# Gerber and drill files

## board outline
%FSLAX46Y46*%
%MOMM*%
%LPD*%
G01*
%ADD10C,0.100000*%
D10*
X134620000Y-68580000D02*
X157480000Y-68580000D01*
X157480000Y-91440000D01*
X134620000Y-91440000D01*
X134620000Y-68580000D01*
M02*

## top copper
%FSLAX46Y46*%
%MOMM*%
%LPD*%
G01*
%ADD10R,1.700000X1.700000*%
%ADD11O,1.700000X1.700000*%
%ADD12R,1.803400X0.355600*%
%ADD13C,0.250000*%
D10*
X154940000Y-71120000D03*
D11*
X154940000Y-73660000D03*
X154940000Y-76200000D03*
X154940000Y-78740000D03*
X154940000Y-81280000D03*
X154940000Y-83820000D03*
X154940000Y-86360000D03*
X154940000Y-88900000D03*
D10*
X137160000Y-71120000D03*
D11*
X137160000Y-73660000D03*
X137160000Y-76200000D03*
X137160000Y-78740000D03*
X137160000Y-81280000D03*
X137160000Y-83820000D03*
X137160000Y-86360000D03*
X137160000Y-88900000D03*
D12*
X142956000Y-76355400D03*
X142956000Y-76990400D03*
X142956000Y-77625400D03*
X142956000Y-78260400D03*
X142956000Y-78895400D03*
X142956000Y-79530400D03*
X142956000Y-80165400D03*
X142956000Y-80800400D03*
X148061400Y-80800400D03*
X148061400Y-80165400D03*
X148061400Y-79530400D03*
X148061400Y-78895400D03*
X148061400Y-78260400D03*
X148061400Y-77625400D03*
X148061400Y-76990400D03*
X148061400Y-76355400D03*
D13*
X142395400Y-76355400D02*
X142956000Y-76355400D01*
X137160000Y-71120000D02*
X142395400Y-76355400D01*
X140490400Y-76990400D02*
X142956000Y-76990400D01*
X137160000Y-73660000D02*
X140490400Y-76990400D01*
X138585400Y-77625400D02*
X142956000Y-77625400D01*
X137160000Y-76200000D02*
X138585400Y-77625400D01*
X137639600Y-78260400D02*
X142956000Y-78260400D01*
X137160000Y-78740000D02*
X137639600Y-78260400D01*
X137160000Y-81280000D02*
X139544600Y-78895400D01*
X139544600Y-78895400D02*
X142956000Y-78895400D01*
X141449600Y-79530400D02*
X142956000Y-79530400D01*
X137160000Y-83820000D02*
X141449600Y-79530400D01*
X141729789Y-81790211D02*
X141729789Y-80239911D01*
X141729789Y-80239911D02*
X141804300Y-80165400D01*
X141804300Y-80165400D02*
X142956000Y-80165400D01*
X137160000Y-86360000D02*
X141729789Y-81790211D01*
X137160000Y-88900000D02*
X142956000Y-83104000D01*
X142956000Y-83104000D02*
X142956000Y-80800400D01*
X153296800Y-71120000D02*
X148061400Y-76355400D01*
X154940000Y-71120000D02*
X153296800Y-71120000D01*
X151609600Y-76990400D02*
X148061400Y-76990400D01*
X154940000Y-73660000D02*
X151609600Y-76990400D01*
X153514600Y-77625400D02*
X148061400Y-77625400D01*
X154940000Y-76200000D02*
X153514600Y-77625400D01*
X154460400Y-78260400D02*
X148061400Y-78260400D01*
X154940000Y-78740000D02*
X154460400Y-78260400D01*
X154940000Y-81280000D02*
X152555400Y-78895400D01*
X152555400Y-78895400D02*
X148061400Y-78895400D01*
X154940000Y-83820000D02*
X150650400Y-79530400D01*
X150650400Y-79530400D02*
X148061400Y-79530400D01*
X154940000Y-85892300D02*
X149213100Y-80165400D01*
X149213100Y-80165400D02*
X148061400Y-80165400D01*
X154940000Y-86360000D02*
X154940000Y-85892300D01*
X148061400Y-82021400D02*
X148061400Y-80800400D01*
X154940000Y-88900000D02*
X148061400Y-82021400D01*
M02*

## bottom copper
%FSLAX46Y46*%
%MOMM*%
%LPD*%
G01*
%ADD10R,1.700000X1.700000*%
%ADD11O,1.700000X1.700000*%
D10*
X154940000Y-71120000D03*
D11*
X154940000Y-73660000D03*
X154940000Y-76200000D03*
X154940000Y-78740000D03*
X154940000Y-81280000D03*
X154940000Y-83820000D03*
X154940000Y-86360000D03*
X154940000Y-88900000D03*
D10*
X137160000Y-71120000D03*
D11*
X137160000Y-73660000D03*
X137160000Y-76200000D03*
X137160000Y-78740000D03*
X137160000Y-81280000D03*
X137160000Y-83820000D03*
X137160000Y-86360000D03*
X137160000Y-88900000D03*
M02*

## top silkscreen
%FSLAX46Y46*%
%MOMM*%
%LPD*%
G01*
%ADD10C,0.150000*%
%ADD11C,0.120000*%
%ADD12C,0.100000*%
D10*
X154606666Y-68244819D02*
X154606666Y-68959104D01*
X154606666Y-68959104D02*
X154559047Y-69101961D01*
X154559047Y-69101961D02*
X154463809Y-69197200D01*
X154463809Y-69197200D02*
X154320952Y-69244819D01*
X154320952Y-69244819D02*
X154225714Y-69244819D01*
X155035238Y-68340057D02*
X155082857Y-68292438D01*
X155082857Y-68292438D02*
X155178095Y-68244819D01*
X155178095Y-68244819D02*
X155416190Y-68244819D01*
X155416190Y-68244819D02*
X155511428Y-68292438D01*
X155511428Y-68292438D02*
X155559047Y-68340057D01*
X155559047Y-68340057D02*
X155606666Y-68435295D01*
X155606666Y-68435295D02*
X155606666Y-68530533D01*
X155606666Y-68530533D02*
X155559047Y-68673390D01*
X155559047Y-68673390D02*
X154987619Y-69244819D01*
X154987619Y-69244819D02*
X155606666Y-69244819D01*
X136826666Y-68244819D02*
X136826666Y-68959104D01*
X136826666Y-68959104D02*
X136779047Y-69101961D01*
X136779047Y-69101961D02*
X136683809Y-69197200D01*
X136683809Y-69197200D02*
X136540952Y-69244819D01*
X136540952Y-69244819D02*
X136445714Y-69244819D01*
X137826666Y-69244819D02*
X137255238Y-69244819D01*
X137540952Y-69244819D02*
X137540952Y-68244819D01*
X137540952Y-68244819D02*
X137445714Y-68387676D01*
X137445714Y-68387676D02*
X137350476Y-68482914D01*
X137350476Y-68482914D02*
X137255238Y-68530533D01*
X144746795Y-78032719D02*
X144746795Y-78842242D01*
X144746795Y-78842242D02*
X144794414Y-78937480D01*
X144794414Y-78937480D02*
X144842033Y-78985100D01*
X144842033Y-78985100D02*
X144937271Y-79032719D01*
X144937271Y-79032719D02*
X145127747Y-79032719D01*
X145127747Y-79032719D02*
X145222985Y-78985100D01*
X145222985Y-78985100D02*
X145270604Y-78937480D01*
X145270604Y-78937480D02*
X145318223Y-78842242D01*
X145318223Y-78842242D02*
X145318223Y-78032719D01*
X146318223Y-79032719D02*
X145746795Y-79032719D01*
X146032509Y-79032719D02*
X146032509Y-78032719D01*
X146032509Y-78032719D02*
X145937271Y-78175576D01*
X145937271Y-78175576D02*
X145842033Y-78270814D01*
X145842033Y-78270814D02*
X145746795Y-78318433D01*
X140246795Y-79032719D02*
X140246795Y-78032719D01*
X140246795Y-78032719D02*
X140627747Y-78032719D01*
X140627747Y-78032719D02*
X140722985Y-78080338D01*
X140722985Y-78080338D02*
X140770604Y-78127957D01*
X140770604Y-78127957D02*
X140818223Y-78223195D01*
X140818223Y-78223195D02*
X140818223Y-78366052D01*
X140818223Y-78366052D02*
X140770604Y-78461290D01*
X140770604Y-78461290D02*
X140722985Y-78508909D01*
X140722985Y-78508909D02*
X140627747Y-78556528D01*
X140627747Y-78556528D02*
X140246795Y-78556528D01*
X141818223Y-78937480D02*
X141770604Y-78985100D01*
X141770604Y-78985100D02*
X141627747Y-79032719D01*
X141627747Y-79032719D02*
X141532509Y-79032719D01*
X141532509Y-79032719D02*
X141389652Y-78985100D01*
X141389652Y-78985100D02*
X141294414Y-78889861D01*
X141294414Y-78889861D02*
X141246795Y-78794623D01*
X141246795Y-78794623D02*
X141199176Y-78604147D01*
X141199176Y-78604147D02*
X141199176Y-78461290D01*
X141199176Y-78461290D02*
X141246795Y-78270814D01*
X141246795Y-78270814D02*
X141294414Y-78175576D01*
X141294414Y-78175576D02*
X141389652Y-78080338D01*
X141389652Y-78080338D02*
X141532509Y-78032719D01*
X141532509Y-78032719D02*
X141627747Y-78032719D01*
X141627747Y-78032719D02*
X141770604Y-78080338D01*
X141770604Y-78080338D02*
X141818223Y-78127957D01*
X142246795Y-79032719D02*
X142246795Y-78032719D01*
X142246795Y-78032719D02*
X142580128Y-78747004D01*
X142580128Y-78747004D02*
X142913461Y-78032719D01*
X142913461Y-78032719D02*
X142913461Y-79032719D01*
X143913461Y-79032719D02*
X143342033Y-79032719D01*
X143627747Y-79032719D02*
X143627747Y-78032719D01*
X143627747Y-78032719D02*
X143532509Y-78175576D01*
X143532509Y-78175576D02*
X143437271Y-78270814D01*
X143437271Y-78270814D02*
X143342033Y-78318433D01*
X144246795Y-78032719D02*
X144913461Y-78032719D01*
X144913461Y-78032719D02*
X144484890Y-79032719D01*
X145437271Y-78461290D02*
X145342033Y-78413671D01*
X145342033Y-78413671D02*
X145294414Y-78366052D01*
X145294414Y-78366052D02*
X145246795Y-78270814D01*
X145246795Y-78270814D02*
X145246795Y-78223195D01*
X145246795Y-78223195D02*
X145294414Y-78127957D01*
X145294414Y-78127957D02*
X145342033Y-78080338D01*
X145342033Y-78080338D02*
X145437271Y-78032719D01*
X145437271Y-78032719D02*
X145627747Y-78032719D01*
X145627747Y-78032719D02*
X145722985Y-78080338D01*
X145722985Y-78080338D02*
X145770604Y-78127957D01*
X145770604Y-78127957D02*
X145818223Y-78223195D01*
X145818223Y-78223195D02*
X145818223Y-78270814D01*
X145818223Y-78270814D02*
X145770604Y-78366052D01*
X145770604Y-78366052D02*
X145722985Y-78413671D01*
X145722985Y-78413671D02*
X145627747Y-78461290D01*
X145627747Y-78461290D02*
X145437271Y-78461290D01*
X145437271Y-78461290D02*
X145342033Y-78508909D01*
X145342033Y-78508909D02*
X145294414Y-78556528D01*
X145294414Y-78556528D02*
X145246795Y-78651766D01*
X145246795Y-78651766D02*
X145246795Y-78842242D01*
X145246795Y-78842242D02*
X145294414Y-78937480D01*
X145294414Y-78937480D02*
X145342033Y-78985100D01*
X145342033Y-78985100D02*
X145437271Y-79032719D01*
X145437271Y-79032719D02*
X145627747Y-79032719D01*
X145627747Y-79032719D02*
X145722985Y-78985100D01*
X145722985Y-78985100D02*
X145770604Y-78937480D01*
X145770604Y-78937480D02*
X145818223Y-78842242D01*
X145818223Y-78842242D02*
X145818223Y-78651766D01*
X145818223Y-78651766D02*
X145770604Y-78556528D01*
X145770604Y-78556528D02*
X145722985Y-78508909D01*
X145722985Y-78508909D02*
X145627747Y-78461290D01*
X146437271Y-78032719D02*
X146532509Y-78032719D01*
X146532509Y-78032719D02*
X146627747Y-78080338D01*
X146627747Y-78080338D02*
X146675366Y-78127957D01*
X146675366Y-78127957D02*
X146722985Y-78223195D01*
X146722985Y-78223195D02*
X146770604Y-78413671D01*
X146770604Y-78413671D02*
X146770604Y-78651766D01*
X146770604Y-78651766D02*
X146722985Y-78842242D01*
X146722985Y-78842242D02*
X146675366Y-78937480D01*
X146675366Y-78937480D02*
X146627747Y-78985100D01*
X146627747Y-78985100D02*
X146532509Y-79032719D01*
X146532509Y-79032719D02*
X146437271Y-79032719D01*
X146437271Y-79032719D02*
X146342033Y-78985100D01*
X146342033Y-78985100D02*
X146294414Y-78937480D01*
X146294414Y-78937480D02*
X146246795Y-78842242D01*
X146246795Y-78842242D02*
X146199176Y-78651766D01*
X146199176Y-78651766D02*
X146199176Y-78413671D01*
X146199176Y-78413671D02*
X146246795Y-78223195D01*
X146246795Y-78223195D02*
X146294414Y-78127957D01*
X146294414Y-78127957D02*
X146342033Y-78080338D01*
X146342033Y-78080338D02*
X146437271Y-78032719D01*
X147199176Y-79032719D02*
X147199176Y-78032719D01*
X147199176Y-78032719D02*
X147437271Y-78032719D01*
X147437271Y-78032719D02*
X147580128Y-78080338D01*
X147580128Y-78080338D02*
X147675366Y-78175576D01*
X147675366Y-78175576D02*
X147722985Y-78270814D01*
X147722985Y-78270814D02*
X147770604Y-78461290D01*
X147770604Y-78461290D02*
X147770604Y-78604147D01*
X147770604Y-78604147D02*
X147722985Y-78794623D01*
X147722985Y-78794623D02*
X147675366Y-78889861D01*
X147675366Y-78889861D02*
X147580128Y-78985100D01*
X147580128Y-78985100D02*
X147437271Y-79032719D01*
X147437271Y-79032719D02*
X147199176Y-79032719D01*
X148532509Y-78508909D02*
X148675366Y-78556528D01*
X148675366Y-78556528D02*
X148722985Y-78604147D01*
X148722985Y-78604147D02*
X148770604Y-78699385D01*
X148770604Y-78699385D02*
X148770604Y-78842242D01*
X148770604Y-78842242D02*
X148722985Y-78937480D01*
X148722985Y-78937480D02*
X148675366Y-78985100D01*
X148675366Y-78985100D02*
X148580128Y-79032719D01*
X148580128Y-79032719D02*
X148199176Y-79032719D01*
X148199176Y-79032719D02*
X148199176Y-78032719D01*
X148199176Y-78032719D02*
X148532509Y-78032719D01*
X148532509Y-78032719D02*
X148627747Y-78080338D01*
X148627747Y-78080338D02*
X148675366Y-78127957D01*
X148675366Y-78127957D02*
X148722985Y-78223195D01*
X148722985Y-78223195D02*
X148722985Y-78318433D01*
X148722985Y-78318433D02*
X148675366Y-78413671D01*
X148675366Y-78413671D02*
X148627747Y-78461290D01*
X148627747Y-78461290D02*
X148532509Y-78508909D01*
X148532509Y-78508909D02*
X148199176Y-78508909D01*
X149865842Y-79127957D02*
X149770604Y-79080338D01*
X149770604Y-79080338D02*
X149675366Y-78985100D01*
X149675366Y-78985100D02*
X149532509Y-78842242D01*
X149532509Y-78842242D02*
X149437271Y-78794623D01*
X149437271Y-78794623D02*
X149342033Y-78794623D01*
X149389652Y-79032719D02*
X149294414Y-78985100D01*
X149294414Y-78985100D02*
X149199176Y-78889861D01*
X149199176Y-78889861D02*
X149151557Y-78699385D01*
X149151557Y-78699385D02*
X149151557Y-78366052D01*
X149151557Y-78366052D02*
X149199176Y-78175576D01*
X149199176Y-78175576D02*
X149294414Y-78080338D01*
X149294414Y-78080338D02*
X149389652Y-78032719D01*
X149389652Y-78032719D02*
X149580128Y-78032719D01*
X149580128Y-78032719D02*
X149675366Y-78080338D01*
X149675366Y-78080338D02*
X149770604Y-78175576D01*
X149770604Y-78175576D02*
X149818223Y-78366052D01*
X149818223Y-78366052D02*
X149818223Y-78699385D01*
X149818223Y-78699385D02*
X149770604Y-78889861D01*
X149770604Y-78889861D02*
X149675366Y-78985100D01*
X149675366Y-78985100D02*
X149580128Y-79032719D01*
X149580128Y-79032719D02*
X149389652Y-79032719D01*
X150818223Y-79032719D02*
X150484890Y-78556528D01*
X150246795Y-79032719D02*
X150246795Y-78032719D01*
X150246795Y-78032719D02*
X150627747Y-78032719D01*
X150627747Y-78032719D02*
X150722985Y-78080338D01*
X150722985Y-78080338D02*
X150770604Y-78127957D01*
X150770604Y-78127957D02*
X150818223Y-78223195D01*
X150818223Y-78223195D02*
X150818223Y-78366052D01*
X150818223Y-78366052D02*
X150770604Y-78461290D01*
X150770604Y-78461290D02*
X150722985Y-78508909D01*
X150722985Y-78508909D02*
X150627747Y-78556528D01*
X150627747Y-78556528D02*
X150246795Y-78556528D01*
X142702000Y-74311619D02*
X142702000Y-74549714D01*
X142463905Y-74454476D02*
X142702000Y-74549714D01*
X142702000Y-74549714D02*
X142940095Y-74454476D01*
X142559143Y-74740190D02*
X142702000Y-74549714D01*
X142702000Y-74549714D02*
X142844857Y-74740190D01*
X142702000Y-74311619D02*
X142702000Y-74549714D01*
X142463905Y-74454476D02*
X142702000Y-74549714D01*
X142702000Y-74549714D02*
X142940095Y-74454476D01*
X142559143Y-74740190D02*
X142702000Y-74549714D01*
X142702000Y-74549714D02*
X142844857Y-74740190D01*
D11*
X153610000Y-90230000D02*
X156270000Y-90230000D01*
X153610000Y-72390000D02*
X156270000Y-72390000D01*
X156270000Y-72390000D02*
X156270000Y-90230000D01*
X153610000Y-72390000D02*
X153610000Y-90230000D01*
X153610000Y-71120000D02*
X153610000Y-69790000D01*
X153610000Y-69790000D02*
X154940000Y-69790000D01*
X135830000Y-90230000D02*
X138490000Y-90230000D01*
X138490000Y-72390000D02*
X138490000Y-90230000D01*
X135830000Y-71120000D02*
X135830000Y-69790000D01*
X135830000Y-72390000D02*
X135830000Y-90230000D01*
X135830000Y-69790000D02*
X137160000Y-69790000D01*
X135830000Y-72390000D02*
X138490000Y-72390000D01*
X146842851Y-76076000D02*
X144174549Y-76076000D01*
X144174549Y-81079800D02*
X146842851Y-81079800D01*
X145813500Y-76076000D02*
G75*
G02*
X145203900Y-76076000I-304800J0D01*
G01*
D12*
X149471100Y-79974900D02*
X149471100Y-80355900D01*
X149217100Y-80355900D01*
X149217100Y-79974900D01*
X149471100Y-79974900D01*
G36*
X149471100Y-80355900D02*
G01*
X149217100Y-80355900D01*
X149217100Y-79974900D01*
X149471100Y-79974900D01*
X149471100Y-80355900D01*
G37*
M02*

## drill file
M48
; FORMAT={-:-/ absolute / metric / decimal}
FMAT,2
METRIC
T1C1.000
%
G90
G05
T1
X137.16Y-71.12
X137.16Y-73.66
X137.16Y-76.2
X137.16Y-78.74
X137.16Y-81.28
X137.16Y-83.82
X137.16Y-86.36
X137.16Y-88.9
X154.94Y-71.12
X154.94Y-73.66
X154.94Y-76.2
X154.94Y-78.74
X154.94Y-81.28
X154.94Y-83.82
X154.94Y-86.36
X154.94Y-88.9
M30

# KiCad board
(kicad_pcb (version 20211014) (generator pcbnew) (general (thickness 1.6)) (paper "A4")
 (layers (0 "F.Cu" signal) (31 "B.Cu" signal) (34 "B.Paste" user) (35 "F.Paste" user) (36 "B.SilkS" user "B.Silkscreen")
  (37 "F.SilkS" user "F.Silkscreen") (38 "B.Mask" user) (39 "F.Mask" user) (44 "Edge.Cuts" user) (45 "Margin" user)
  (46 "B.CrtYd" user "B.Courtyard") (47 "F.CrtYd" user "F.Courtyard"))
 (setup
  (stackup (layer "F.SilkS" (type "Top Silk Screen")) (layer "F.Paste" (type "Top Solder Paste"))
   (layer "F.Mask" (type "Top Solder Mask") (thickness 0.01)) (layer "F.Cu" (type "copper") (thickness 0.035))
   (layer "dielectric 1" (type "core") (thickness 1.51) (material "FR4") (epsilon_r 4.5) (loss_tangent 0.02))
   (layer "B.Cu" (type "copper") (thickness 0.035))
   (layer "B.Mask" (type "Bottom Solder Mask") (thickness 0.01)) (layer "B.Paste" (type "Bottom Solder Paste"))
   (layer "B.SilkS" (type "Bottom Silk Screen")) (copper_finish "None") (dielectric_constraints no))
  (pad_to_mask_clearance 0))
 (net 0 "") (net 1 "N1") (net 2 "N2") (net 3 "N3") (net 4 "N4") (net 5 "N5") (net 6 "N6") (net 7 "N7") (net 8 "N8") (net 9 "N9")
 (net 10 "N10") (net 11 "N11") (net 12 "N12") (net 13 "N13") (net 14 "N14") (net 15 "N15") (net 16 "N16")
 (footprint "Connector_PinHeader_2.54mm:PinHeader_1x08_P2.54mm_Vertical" (layer "F.Cu") (at 154.94 71.12)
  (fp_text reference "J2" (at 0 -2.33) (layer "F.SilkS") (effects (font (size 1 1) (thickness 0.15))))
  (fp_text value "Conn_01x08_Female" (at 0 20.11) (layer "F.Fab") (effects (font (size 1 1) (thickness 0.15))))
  (fp_line (start -1.33 19.11) (end 1.33 19.11) (layer "F.SilkS") (width 0.12))
  (fp_line (start -1.33 1.27) (end 1.33 1.27) (layer "F.SilkS") (width 0.12))
  (fp_line (start 1.33 1.27) (end 1.33 19.11) (layer "F.SilkS") (width 0.12))
  (fp_line (start -1.33 1.27) (end -1.33 19.11) (layer "F.SilkS") (width 0.12))
  (fp_line (start -1.33 0) (end -1.33 -1.33) (layer "F.SilkS") (width 0.12))
  (fp_line (start -1.33 -1.33) (end 0 -1.33) (layer "F.SilkS") (width 0.12))
  (pad "1" thru_hole rect (at 0 0) (size 1.7 1.7) (drill 1) (layers *.Cu *.Mask) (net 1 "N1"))
  (pad "2" thru_hole oval (at 0 2.54) (size 1.7 1.7) (drill 1) (layers *.Cu *.Mask) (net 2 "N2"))
  (pad "3" thru_hole oval (at 0 5.08) (size 1.7 1.7) (drill 1) (layers *.Cu *.Mask) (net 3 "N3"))
  (pad "4" thru_hole oval (at 0 7.62) (size 1.7 1.7) (drill 1) (layers *.Cu *.Mask) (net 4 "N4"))
  (pad "5" thru_hole oval (at 0 10.16) (size 1.7 1.7) (drill 1) (layers *.Cu *.Mask) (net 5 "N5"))
  (pad "6" thru_hole oval (at 0 12.7) (size 1.7 1.7) (drill 1) (layers *.Cu *.Mask) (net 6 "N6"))
  (pad "7" thru_hole oval (at 0 15.24) (size 1.7 1.7) (drill 1) (layers *.Cu *.Mask) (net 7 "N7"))
  (pad "8" thru_hole oval (at 0 17.78) (size 1.7 1.7) (drill 1) (layers *.Cu *.Mask) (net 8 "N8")))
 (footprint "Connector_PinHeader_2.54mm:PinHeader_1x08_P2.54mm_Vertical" (layer "F.Cu") (at 137.16 71.12)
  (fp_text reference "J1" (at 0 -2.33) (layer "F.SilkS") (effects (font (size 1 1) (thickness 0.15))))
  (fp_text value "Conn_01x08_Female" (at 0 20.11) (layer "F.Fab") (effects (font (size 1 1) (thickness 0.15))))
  (fp_line (start -1.33 19.11) (end 1.33 19.11) (layer "F.SilkS") (width 0.12))
  (fp_line (start 1.33 1.27) (end 1.33 19.11) (layer "F.SilkS") (width 0.12))
  (fp_line (start -1.33 0) (end -1.33 -1.33) (layer "F.SilkS") (width 0.12))
  (fp_line (start -1.33 1.27) (end -1.33 19.11) (layer "F.SilkS") (width 0.12))
  (fp_line (start -1.33 -1.33) (end 0 -1.33) (layer "F.SilkS") (width 0.12))
  (fp_line (start -1.33 1.27) (end 1.33 1.27) (layer "F.SilkS") (width 0.12))
  (pad "1" thru_hole rect (at 0 0) (size 1.7 1.7) (drill 1) (layers *.Cu *.Mask) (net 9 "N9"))
  (pad "2" thru_hole oval (at 0 2.54) (size 1.7 1.7) (drill 1) (layers *.Cu *.Mask) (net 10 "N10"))
  (pad "3" thru_hole oval (at 0 5.08) (size 1.7 1.7) (drill 1) (layers *.Cu *.Mask) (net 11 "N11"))
  (pad "4" thru_hole oval (at 0 7.62) (size 1.7 1.7) (drill 1) (layers *.Cu *.Mask) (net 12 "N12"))
  (pad "5" thru_hole oval (at 0 10.16) (size 1.7 1.7) (drill 1) (layers *.Cu *.Mask) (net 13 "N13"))
  (pad "6" thru_hole oval (at 0 12.7) (size 1.7 1.7) (drill 1) (layers *.Cu *.Mask) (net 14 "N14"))
  (pad "7" thru_hole oval (at 0 15.24) (size 1.7 1.7) (drill 1) (layers *.Cu *.Mask) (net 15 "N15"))
  (pad "8" thru_hole oval (at 0 17.78) (size 1.7 1.7) (drill 1) (layers *.Cu *.Mask) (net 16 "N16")))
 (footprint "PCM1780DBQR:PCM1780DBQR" (layer "F.Cu") (at 145.5087 78.5779)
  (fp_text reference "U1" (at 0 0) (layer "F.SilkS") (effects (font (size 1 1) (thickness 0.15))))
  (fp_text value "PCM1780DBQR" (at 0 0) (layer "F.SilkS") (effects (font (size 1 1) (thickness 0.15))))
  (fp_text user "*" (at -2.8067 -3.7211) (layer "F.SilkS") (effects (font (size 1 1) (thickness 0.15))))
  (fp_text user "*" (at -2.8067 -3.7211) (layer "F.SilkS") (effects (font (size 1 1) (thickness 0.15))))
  (fp_line (start 1.334151 -2.5019) (end -1.334151 -2.5019) (layer "F.SilkS") (width 0.12))
  (fp_line (start -1.334151 2.5019) (end 1.334151 2.5019) (layer "F.SilkS") (width 0.12))
  (fp_arc (start 0.3048 -2.5019) (mid 0 -2.1971) (end -0.3048 -2.5019) (layer "F.SilkS") (width 0.12))
  (fp_poly (pts (xy 3.9624 1.397) (xy 3.9624 1.778) (xy 3.7084 1.778) (xy 3.7084 1.397)) (layer "F.SilkS") (width 0.1) (fill solid))
  (pad "1" smd rect (at -2.5527 -2.2225) (size 1.8034 0.3556) (layers "F.Cu" "F.Paste" "F.Mask") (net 9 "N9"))
  (pad "2" smd rect (at -2.5527 -1.5875) (size 1.8034 0.3556) (layers "F.Cu" "F.Paste" "F.Mask") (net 10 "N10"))
  (pad "3" smd rect (at -2.5527 -0.9525) (size 1.8034 0.3556) (layers "F.Cu" "F.Paste" "F.Mask") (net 11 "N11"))
  (pad "4" smd rect (at -2.5527 -0.3175) (size 1.8034 0.3556) (layers "F.Cu" "F.Paste" "F.Mask") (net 12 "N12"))
  (pad "5" smd rect (at -2.5527 0.3175) (size 1.8034 0.3556) (layers "F.Cu" "F.Paste" "F.Mask") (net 13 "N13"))
  (pad "6" smd rect (at -2.5527 0.9525) (size 1.8034 0.3556) (layers "F.Cu" "F.Paste" "F.Mask") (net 14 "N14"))
  (pad "7" smd rect (at -2.5527 1.5875) (size 1.8034 0.3556) (layers "F.Cu" "F.Paste" "F.Mask") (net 15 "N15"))
  (pad "8" smd rect (at -2.5527 2.2225) (size 1.8034 0.3556) (layers "F.Cu" "F.Paste" "F.Mask") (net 16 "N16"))
  (pad "9" smd rect (at 2.5527 2.2225) (size 1.8034 0.3556) (layers "F.Cu" "F.Paste" "F.Mask") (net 8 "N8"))
  (pad "10" smd rect (at 2.5527 1.5875) (size 1.8034 0.3556) (layers "F.Cu" "F.Paste" "F.Mask") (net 7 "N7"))
  (pad "11" smd rect (at 2.5527 0.9525) (size 1.8034 0.3556) (layers "F.Cu" "F.Paste" "F.Mask") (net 6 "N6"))
  (pad "12" smd rect (at 2.5527 0.3175) (size 1.8034 0.3556) (layers "F.Cu" "F.Paste" "F.Mask") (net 5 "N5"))
  (pad "13" smd rect (at 2.5527 -0.3175) (size 1.8034 0.3556) (layers "F.Cu" "F.Paste" "F.Mask") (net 4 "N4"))
  (pad "14" smd rect (at 2.5527 -0.9525) (size 1.8034 0.3556) (layers "F.Cu" "F.Paste" "F.Mask") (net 3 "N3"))
  (pad "15" smd rect (at 2.5527 -1.5875) (size 1.8034 0.3556) (layers "F.Cu" "F.Paste" "F.Mask") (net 2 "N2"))
  (pad "16" smd rect (at 2.5527 -2.2225) (size 1.8034 0.3556) (layers "F.Cu" "F.Paste" "F.Mask") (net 1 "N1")))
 (gr_rect (start 134.62 68.58) (end 157.48 91.44) (layer "Edge.Cuts") (width 0.1) (fill none))
 (segment (start 142.3954 76.3554) (end 142.956 76.3554) (width 0.25) (layer "F.Cu") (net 9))
 (segment (start 137.16 71.12) (end 142.3954 76.3554) (width 0.25) (layer "F.Cu") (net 9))
 (segment (start 140.4904 76.9904) (end 142.956 76.9904) (width 0.25) (layer "F.Cu") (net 10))
 (segment (start 137.16 73.66) (end 140.4904 76.9904) (width 0.25) (layer "F.Cu") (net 10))
 (segment (start 138.5854 77.6254) (end 142.956 77.6254) (width 0.25) (layer "F.Cu") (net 11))
 (segment (start 137.16 76.2) (end 138.5854 77.6254) (width 0.25) (layer "F.Cu") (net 11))
 (segment (start 137.6396 78.2604) (end 142.956 78.2604) (width 0.25) (layer "F.Cu") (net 12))
 (segment (start 137.16 78.74) (end 137.6396 78.2604) (width 0.25) (layer "F.Cu") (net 12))
 (segment (start 137.16 81.28) (end 139.5446 78.8954) (width 0.25) (layer "F.Cu") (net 13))
 (segment (start 139.5446 78.8954) (end 142.956 78.8954) (width 0.25) (layer "F.Cu") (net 13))
 (segment (start 141.4496 79.5304) (end 142.956 79.5304) (width 0.25) (layer "F.Cu") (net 14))
 (segment (start 137.16 83.82) (end 141.4496 79.5304) (width 0.25) (layer "F.Cu") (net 14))
 (segment (start 141.729789 81.790211) (end 141.729789 80.239911) (width 0.25) (layer "F.Cu") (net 15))
 (segment (start 141.729789 80.239911) (end 141.8043 80.1654) (width 0.25) (layer "F.Cu") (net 15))
 (segment (start 141.8043 80.1654) (end 142.956 80.1654) (width 0.25) (layer "F.Cu") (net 15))
 (segment (start 137.16 86.36) (end 141.729789 81.790211) (width 0.25) (layer "F.Cu") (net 15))
 (segment (start 137.16 88.9) (end 142.956 83.104) (width 0.25) (layer "F.Cu") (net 16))
 (segment (start 142.956 83.104) (end 142.956 80.8004) (width 0.25) (layer "F.Cu") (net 16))
 (segment (start 153.2968 71.12) (end 148.0614 76.3554) (width 0.25) (layer "F.Cu") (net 1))
 (segment (start 154.94 71.12) (end 153.2968 71.12) (width 0.25) (layer "F.Cu") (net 1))
 (segment (start 151.6096 76.9904) (end 148.0614 76.9904) (width 0.25) (layer "F.Cu") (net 2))
 (segment (start 154.94 73.66) (end 151.6096 76.9904) (width 0.25) (layer "F.Cu") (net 2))
 (segment (start 153.5146 77.6254) (end 148.0614 77.6254) (width 0.25) (layer "F.Cu") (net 3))
 (segment (start 154.94 76.2) (end 153.5146 77.6254) (width 0.25) (layer "F.Cu") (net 3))
 (segment (start 154.4604 78.2604) (end 148.0614 78.2604) (width 0.25) (layer "F.Cu") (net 4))
 (segment (start 154.94 78.74) (end 154.4604 78.2604) (width 0.25) (layer "F.Cu") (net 4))
 (segment (start 154.94 81.28) (end 152.5554 78.8954) (width 0.25) (layer "F.Cu") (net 5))
 (segment (start 152.5554 78.8954) (end 148.0614 78.8954) (width 0.25) (layer "F.Cu") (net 5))
 (segment (start 154.94 83.82) (end 150.6504 79.5304) (width 0.25) (layer "F.Cu") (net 6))
 (segment (start 150.6504 79.5304) (end 148.0614 79.5304) (width 0.25) (layer "F.Cu") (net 6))
 (segment (start 154.94 85.8923) (end 149.2131 80.1654) (width 0.25) (layer "F.Cu") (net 7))
 (segment (start 149.2131 80.1654) (end 148.0614 80.1654) (width 0.25) (layer "F.Cu") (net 7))
 (segment (start 154.94 86.36) (end 154.94 85.8923) (width 0.25) (layer "F.Cu") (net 7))
 (segment (start 148.0614 82.0214) (end 148.0614 80.8004) (width 0.25) (layer "F.Cu") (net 8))
 (segment (start 154.94 88.9) (end 148.0614 82.0214) (width 0.25) (layer "F.Cu") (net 8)))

